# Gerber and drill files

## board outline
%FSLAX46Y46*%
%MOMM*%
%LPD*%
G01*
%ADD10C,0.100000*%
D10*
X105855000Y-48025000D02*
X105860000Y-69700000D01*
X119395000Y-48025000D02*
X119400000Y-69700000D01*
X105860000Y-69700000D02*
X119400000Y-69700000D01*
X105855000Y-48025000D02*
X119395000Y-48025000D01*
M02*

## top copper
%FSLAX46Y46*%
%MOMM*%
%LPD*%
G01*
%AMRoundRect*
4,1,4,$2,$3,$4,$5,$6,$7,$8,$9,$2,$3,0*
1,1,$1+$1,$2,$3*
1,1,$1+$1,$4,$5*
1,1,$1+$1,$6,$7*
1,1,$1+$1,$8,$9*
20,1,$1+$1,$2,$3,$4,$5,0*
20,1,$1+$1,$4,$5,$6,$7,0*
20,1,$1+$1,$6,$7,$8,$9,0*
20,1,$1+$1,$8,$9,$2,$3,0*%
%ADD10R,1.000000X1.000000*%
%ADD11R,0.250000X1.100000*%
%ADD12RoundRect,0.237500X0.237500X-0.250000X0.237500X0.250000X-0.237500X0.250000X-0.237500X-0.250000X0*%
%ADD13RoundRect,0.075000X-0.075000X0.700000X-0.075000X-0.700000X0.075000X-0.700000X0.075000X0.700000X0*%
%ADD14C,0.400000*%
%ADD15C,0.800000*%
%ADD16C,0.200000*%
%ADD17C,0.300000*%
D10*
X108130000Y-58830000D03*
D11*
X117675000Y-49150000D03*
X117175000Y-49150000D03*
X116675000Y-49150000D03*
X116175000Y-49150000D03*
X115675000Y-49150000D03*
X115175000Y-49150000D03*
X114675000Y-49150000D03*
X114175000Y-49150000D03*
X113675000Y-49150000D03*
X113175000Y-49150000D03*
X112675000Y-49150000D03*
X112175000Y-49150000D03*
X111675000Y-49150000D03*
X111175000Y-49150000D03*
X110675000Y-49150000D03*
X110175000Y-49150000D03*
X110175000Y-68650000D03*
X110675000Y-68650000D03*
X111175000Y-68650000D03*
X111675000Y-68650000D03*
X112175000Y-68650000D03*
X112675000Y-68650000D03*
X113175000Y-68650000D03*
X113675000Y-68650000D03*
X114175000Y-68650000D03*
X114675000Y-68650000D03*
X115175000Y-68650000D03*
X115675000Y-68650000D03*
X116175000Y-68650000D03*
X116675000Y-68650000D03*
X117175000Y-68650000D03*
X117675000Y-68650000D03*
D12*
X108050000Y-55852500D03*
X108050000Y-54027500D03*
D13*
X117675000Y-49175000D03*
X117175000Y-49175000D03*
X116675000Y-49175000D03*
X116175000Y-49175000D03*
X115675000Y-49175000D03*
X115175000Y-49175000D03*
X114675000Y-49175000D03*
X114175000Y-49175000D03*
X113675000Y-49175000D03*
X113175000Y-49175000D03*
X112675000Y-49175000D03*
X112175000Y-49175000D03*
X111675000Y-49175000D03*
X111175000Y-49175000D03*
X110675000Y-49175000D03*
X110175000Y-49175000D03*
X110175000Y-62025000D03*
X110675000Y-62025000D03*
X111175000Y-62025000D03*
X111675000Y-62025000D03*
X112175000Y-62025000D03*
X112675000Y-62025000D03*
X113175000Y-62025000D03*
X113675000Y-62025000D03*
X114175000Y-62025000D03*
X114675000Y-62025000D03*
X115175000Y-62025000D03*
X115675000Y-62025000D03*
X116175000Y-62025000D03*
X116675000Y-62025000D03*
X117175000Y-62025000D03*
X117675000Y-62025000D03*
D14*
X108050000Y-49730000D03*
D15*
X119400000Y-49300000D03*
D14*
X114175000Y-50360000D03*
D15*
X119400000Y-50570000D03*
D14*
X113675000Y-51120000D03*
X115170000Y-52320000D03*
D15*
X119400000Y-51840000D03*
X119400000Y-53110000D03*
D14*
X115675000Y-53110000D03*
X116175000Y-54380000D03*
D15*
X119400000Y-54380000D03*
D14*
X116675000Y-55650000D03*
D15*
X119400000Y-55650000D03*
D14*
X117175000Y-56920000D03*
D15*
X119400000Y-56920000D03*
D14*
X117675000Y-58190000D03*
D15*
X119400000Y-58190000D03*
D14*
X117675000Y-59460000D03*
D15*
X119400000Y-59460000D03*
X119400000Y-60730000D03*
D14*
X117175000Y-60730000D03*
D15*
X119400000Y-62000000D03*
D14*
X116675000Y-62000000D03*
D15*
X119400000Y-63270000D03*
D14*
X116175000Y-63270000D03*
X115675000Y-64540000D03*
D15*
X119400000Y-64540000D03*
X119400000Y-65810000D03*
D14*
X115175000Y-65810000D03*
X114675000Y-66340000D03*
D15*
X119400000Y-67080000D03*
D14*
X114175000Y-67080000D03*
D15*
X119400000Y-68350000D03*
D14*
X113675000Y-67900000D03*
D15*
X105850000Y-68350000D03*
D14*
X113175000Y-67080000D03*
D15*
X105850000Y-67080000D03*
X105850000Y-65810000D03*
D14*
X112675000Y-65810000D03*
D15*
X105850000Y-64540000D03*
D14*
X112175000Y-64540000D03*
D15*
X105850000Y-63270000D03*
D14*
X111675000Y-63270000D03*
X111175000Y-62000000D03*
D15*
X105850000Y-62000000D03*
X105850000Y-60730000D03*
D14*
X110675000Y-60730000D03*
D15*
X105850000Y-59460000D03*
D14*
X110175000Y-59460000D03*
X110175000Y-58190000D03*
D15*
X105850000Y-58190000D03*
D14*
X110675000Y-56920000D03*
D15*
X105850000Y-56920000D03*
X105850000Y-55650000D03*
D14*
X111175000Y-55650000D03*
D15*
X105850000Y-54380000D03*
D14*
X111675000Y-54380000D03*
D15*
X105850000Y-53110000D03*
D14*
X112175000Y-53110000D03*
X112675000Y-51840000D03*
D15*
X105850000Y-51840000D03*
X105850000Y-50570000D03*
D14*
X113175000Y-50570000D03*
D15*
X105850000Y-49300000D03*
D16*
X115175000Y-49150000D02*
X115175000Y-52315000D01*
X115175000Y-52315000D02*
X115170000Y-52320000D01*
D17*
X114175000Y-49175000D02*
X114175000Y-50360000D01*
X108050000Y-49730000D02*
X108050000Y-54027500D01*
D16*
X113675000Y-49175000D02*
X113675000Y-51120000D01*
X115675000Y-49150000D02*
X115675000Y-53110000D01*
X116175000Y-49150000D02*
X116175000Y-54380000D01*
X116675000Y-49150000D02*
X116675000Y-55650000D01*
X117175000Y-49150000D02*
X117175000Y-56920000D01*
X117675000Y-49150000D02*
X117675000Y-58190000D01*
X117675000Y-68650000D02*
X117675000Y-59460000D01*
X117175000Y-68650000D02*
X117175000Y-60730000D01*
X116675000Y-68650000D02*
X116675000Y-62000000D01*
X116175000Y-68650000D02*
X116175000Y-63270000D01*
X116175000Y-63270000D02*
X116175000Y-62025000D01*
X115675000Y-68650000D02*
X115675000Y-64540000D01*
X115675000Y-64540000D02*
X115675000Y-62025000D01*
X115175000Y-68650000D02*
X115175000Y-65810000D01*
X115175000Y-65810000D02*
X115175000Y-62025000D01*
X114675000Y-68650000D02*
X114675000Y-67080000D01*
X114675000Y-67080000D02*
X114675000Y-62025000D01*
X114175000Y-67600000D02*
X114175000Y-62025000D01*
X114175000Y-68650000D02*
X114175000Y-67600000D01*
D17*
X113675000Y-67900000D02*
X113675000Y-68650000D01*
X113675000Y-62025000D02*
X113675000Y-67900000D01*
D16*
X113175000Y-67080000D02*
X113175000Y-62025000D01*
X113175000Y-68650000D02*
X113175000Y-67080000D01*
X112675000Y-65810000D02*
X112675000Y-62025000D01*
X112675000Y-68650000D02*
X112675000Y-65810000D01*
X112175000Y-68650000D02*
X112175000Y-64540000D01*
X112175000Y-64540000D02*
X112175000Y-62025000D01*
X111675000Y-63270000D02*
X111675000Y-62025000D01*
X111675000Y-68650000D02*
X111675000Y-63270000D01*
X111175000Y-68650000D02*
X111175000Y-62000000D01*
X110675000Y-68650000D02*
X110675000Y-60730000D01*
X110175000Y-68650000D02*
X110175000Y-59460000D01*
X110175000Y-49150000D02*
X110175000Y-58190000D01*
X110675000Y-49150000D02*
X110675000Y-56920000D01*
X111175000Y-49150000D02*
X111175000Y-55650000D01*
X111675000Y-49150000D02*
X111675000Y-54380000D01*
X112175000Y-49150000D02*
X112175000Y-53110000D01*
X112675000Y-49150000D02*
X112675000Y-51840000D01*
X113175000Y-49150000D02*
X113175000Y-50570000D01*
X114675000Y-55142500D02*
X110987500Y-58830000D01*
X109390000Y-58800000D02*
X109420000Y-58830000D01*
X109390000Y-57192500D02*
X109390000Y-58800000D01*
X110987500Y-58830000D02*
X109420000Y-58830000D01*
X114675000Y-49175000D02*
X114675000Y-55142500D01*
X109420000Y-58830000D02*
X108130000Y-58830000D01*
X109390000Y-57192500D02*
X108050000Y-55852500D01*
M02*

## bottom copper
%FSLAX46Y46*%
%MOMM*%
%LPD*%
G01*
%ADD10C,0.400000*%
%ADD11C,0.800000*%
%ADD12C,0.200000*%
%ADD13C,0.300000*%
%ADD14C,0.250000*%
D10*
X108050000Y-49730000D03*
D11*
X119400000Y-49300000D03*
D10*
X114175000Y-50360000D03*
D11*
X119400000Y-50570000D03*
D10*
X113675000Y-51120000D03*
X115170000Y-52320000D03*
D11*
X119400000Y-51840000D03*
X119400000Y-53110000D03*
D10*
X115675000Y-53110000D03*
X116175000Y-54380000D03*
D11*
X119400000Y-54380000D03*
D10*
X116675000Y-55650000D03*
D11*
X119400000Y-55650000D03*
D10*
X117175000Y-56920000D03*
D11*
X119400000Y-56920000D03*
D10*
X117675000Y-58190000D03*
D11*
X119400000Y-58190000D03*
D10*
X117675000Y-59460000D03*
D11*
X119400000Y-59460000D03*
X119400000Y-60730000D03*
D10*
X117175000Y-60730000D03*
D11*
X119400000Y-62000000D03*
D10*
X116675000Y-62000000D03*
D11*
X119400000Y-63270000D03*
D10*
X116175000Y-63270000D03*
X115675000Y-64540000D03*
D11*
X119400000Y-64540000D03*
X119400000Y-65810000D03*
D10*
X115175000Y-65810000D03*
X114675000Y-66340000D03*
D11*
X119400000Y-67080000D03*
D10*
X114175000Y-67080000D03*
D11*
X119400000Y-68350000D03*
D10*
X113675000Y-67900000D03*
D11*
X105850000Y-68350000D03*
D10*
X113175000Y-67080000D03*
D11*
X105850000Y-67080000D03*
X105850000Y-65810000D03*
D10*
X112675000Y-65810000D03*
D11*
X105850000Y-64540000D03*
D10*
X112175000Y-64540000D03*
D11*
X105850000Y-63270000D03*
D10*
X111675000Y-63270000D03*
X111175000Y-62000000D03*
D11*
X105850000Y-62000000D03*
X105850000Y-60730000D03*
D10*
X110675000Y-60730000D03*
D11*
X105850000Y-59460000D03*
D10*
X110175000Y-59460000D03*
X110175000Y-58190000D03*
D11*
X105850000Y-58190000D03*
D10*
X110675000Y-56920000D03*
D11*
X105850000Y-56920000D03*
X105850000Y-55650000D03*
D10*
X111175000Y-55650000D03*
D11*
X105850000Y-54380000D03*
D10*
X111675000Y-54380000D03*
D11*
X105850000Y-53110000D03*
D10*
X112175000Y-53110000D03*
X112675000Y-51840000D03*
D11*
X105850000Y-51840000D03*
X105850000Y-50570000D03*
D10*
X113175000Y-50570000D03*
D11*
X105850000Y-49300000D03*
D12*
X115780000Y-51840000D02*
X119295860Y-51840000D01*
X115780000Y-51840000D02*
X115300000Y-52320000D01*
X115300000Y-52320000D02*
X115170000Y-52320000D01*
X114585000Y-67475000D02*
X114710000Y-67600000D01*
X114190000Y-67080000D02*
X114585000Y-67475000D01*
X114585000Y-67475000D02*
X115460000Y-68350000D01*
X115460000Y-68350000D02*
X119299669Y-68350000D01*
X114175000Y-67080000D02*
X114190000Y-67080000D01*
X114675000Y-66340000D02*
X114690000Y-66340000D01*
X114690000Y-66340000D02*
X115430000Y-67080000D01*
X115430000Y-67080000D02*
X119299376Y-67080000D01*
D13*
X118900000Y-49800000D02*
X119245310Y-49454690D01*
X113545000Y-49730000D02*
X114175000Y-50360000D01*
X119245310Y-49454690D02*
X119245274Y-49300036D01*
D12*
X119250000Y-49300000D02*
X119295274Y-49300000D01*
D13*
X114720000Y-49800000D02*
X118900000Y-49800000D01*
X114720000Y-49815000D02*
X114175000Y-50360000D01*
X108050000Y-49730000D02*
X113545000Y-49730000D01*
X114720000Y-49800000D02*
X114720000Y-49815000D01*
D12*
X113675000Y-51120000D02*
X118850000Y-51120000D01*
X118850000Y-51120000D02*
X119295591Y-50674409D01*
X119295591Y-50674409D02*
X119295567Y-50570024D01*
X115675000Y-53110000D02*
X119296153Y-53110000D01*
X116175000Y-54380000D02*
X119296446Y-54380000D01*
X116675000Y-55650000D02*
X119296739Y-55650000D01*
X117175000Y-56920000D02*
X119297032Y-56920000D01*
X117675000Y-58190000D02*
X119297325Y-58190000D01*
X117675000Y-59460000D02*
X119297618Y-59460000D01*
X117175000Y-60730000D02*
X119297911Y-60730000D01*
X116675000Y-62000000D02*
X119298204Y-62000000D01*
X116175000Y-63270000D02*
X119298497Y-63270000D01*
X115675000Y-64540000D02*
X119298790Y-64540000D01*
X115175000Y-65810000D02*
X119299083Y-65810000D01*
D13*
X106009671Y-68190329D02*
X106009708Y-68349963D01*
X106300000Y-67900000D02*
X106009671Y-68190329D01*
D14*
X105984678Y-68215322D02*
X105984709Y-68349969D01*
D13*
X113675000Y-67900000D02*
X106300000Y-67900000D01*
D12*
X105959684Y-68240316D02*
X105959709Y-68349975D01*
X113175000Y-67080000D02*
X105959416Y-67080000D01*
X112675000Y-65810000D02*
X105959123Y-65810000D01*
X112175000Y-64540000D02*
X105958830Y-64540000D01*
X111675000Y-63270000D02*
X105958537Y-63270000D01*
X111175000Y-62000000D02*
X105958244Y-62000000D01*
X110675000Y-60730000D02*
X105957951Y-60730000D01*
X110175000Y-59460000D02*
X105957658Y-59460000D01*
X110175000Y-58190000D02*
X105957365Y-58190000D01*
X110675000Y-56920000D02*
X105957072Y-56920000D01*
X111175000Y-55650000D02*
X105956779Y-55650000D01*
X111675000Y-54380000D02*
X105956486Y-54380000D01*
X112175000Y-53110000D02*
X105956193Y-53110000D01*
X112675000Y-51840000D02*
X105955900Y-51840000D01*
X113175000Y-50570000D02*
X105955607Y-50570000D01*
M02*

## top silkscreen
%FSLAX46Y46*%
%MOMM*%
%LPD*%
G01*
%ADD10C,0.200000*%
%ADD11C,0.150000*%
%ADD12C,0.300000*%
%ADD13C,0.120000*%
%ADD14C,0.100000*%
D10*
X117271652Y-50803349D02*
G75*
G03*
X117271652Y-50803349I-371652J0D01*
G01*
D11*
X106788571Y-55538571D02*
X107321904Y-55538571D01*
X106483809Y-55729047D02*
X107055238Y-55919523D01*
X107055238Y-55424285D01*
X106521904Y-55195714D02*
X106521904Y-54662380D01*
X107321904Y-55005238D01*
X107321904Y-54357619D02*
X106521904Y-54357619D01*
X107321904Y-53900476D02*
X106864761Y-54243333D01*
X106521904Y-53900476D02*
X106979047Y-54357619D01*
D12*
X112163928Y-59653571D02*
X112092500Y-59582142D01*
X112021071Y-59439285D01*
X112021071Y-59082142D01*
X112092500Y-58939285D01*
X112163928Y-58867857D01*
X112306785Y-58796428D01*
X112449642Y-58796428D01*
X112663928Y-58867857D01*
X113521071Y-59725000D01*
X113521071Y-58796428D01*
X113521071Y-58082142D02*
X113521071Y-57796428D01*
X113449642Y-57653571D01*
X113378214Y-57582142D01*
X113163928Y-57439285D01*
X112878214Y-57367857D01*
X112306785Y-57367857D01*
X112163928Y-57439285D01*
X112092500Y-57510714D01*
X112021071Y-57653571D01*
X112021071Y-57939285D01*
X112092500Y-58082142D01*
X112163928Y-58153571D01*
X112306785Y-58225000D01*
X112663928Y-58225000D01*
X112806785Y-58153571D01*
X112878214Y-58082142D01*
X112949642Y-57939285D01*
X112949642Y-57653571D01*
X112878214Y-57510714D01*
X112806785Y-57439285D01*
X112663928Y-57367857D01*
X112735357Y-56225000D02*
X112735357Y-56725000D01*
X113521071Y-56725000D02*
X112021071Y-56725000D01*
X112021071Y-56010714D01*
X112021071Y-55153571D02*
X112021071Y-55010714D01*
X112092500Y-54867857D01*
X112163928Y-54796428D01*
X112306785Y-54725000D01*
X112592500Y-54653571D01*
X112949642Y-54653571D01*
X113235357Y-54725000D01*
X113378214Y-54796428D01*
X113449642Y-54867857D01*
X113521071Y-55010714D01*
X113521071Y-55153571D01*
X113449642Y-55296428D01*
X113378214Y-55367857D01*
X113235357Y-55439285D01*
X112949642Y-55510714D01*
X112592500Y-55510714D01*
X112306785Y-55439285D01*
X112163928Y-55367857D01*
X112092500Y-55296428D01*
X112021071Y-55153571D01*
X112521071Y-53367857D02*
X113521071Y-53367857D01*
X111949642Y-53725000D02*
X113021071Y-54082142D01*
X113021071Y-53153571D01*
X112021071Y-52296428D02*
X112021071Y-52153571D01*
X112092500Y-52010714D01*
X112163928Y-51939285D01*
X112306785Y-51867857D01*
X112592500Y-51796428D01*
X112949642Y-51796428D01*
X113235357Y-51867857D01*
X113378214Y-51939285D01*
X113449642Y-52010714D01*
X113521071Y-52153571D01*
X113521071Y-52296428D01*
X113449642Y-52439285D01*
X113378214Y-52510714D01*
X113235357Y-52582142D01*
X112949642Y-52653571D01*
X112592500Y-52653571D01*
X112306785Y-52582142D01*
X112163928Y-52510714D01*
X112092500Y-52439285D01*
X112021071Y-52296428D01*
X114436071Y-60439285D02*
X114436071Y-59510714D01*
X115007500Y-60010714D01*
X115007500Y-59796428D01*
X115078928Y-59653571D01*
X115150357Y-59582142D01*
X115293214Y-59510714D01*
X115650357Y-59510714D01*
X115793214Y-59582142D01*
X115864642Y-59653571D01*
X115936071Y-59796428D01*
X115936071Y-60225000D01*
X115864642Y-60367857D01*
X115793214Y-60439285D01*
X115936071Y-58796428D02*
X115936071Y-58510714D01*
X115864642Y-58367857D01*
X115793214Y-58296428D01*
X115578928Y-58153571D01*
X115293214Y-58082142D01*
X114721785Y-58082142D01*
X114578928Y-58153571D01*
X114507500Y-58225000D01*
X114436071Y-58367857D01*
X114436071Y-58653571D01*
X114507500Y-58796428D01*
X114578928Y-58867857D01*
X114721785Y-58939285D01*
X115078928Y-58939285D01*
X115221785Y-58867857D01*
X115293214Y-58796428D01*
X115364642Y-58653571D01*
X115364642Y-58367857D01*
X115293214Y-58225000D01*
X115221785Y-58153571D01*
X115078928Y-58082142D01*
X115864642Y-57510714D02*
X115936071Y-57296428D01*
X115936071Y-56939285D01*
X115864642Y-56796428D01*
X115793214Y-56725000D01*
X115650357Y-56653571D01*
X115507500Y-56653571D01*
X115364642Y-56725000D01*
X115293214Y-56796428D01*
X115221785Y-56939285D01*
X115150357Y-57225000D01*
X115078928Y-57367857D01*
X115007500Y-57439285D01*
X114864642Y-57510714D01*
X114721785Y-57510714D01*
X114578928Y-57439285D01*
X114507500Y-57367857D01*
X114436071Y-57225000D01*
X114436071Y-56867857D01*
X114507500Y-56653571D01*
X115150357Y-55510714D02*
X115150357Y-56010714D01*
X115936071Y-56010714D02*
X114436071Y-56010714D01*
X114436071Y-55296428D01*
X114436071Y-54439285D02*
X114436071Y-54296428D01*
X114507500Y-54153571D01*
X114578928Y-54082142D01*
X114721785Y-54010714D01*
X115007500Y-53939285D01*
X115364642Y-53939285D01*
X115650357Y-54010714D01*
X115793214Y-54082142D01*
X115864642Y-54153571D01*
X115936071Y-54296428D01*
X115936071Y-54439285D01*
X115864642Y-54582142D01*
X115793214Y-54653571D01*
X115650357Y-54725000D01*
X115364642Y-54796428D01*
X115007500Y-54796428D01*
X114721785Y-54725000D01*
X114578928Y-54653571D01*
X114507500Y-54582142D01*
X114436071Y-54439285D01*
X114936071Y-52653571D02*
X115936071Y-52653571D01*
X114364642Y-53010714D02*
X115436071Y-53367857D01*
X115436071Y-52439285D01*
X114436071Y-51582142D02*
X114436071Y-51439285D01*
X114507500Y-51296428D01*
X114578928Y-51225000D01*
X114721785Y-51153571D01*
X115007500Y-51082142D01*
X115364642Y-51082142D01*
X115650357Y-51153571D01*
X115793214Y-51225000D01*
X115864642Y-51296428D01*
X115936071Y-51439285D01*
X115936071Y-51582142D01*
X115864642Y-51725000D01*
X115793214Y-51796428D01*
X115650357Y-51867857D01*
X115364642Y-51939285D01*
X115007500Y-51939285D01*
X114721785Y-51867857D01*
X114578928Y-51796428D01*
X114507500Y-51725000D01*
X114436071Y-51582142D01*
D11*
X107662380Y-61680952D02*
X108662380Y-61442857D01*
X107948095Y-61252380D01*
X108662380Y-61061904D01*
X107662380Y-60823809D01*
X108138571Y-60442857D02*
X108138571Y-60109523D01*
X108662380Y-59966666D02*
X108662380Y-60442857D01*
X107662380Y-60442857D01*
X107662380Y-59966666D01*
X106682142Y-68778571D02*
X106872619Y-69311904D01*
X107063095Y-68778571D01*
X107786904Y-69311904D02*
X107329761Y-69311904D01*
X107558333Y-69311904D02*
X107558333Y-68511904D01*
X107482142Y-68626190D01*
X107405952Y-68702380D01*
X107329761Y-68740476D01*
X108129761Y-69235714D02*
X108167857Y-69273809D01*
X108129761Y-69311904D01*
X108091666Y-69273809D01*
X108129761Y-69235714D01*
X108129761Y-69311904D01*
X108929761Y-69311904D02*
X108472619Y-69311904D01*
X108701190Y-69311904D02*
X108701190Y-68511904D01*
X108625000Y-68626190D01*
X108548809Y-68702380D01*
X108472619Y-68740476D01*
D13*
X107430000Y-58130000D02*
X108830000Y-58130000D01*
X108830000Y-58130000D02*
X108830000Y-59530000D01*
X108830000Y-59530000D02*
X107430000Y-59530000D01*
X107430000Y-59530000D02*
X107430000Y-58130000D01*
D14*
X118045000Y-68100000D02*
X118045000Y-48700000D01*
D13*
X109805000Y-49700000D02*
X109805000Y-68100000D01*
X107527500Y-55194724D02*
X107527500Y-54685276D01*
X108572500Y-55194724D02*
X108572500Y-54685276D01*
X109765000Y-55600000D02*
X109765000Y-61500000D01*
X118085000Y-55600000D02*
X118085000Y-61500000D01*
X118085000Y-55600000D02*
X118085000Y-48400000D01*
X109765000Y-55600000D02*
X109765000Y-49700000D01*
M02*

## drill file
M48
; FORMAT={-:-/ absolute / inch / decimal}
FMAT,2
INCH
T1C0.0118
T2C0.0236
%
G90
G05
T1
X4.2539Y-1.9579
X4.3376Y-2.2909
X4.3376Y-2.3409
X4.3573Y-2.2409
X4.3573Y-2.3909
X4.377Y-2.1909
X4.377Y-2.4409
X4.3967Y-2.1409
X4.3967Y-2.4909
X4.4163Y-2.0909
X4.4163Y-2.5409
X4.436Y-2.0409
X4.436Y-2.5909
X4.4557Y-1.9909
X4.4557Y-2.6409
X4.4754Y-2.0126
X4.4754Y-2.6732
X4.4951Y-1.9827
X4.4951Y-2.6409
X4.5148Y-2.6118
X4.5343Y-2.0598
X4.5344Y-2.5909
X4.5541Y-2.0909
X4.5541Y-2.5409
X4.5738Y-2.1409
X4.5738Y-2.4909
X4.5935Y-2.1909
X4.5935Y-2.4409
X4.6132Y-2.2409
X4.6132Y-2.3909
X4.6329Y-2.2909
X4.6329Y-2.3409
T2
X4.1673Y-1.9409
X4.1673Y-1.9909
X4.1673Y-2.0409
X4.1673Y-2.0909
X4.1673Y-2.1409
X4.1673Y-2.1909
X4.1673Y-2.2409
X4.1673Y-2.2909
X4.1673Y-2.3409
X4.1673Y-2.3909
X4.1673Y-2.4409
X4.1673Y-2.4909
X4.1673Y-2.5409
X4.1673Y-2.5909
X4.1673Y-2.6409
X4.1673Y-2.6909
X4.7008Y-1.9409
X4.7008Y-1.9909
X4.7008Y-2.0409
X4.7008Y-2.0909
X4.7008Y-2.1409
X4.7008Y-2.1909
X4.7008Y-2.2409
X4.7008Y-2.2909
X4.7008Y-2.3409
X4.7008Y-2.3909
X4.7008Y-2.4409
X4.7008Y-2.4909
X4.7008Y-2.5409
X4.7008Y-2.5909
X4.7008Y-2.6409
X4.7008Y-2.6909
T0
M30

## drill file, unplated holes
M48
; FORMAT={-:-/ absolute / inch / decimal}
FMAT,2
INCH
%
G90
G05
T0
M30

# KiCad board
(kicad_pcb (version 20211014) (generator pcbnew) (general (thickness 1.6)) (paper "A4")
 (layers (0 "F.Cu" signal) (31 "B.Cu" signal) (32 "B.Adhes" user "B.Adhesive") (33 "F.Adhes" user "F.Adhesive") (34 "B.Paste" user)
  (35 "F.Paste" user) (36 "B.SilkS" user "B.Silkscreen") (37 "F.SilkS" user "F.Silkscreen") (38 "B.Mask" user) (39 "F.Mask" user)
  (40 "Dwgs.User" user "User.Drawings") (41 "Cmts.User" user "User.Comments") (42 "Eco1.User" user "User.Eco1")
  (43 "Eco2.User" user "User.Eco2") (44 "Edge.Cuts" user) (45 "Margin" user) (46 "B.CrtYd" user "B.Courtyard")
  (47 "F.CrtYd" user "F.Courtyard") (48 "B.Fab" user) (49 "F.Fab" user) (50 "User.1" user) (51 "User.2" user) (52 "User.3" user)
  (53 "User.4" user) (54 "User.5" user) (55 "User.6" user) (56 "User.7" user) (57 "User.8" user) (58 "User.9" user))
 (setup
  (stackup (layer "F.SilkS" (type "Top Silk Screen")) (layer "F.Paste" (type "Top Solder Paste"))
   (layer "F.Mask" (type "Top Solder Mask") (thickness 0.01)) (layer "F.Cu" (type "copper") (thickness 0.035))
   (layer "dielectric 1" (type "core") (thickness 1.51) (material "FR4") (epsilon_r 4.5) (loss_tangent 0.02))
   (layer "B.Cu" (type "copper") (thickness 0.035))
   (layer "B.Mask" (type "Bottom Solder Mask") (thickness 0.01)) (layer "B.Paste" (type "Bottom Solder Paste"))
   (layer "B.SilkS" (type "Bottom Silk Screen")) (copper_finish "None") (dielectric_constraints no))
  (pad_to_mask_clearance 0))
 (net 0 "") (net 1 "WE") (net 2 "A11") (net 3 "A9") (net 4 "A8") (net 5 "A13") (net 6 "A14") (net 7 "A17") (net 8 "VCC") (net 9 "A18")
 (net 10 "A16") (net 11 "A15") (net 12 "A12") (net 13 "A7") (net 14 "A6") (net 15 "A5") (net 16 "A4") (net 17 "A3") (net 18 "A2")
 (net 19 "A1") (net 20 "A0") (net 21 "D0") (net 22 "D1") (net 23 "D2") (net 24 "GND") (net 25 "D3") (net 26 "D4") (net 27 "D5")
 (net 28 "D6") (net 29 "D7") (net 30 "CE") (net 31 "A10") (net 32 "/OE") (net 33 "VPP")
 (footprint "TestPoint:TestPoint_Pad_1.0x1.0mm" (layer "F.Cu") (at 108.13 58.83)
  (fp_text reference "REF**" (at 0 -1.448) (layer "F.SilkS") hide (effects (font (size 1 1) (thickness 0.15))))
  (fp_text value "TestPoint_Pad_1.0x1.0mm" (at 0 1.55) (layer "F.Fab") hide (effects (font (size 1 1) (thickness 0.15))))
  (fp_line (start -0.7 -0.7) (end 0.7 -0.7) (layer "F.SilkS") (width 0.12))
  (fp_line (start 0.7 -0.7) (end 0.7 0.7) (layer "F.SilkS") (width 0.12))
  (fp_line (start 0.7 0.7) (end -0.7 0.7) (layer "F.SilkS") (width 0.12))
  (fp_line (start -0.7 0.7) (end -0.7 -0.7) (layer "F.SilkS") (width 0.12))
  (pad "" smd rect (at 0 0) (size 1 1) (layers "F.Cu" "F.Mask") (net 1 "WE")))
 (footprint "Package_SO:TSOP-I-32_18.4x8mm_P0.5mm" (layer "F.Cu") (at 113.925 58.9 -90)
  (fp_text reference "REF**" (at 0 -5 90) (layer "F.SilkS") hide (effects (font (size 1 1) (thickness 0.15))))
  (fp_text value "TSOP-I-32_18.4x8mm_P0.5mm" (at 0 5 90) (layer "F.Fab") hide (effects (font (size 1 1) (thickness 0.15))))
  (fp_line (start 9.2 -4.12) (end -10.2 -4.12) (layer "F.SilkS") (width 0.1))
  (fp_line (start -9.2 4.12) (end 9.2 4.12) (layer "F.SilkS") (width 0.12))
  (pad "1" smd rect (at -9.75 -3.75 270) (size 1.1 0.25) (layers "F.Cu" "F.Paste" "F.Mask") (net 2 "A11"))
  (pad "2" smd rect (at -9.75 -3.25 270) (size 1.1 0.25) (layers "F.Cu" "F.Paste" "F.Mask") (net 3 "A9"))
  (pad "3" smd rect (at -9.75 -2.75 270) (size 1.1 0.25) (layers "F.Cu" "F.Paste" "F.Mask") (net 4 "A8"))
  (pad "4" smd rect (at -9.75 -2.25 270) (size 1.1 0.25) (layers "F.Cu" "F.Paste" "F.Mask") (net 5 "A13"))
  (pad "5" smd rect (at -9.75 -1.75 270) (size 1.1 0.25) (layers "F.Cu" "F.Paste" "F.Mask") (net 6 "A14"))
  (pad "6" smd rect (at -9.75 -1.25 270) (size 1.1 0.25) (layers "F.Cu" "F.Paste" "F.Mask") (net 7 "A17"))
  (pad "7" smd rect (at -9.75 -0.75 270) (size 1.1 0.25) (layers "F.Cu" "F.Paste" "F.Mask") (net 1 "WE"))
  (pad "8" smd rect (at -9.75 -0.25 270) (size 1.1 0.25) (layers "F.Cu" "F.Paste" "F.Mask") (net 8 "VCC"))
  (pad "9" smd rect (at -9.75 0.25 270) (size 1.1 0.25) (layers "F.Cu" "F.Paste" "F.Mask") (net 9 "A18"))
  (pad "10" smd rect (at -9.75 0.75 270) (size 1.1 0.25) (layers "F.Cu" "F.Paste" "F.Mask") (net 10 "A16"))
  (pad "11" smd rect (at -9.75 1.25 270) (size 1.1 0.25) (layers "F.Cu" "F.Paste" "F.Mask") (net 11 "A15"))
  (pad "12" smd rect (at -9.75 1.75 270) (size 1.1 0.25) (layers "F.Cu" "F.Paste" "F.Mask") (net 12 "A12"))
  (pad "13" smd rect (at -9.75 2.25 270) (size 1.1 0.25) (layers "F.Cu" "F.Paste" "F.Mask") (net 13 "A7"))
  (pad "14" smd rect (at -9.75 2.75 270) (size 1.1 0.25) (layers "F.Cu" "F.Paste" "F.Mask") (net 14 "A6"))
  (pad "15" smd rect (at -9.75 3.25 270) (size 1.1 0.25) (layers "F.Cu" "F.Paste" "F.Mask") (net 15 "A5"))
  (pad "16" smd rect (at -9.75 3.75 270) (size 1.1 0.25) (layers "F.Cu" "F.Paste" "F.Mask") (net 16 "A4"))
  (pad "17" smd rect (at 9.75 3.75 270) (size 1.1 0.25) (layers "F.Cu" "F.Paste" "F.Mask") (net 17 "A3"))
  (pad "18" smd rect (at 9.75 3.25 270) (size 1.1 0.25) (layers "F.Cu" "F.Paste" "F.Mask") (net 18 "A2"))
  (pad "19" smd rect (at 9.75 2.75 270) (size 1.1 0.25) (layers "F.Cu" "F.Paste" "F.Mask") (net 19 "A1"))
  (pad "20" smd rect (at 9.75 2.25 270) (size 1.1 0.25) (layers "F.Cu" "F.Paste" "F.Mask") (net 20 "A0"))
  (pad "21" smd rect (at 9.75 1.75 270) (size 1.1 0.25) (layers "F.Cu" "F.Paste" "F.Mask") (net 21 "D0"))
  (pad "22" smd rect (at 9.75 1.25 270) (size 1.1 0.25) (layers "F.Cu" "F.Paste" "F.Mask") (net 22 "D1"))
  (pad "23" smd rect (at 9.75 0.75 270) (size 1.1 0.25) (layers "F.Cu" "F.Paste" "F.Mask") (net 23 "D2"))
  (pad "24" smd rect (at 9.75 0.25 270) (size 1.1 0.25) (layers "F.Cu" "F.Paste" "F.Mask") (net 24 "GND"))
  (pad "25" smd rect (at 9.75 -0.25 270) (size 1.1 0.25) (layers "F.Cu" "F.Paste" "F.Mask") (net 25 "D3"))
  (pad "26" smd rect (at 9.75 -0.75 270) (size 1.1 0.25) (layers "F.Cu" "F.Paste" "F.Mask") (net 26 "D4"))
  (pad "27" smd rect (at 9.75 -1.25 270) (size 1.1 0.25) (layers "F.Cu" "F.Paste" "F.Mask") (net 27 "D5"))
  (pad "28" smd rect (at 9.75 -1.75 270) (size 1.1 0.25) (layers "F.Cu" "F.Paste" "F.Mask") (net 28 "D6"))
  (pad "29" smd rect (at 9.75 -2.25 270) (size 1.1 0.25) (layers "F.Cu" "F.Paste" "F.Mask") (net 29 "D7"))
  (pad "30" smd rect (at 9.75 -2.75 270) (size 1.1 0.25) (layers "F.Cu" "F.Paste" "F.Mask") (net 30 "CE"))
  (pad "31" smd rect (at 9.75 -3.25 270) (size 1.1 0.25) (layers "F.Cu" "F.Paste" "F.Mask") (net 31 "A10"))
  (pad "32" smd rect (at 9.75 -3.75 270) (size 1.1 0.25) (layers "F.Cu" "F.Paste" "F.Mask") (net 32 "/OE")))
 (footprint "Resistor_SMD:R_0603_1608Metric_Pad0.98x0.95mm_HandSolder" (layer "F.Cu") (at 108.05 54.94 90)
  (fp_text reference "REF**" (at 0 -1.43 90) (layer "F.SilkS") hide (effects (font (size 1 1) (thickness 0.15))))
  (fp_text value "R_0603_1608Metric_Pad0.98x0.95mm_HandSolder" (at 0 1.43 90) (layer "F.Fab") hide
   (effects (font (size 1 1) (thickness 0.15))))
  (fp_line (start -0.254724 -0.5225) (end 0.254724 -0.5225) (layer "F.SilkS") (width 0.12))
  (fp_line (start -0.254724 0.5225) (end 0.254724 0.5225) (layer "F.SilkS") (width 0.12))
  (pad "" smd roundrect (at -0.9125 0 90) (size 0.975 0.95) (layers "F.Cu" "F.Paste" "F.Mask") (roundrect_rratio 0.25) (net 1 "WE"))
  (pad "" smd roundrect (at 0.9125 0 90) (size 0.975 0.95) (layers "F.Cu" "F.Paste" "F.Mask") (roundrect_rratio 0.25) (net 8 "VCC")))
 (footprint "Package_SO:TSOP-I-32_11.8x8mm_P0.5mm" (layer "F.Cu") (at 113.925 55.6 -90)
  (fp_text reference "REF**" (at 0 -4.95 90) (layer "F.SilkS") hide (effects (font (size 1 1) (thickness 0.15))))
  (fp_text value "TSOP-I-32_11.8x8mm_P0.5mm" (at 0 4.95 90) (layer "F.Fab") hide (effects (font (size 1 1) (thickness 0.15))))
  (fp_line (start 0 4.16) (end 5.9 4.16) (layer "F.SilkS") (width 0.12))
  (fp_line (start 0 -4.16) (end 5.9 -4.16) (layer "F.SilkS") (width 0.12))
  (fp_line (start 0 -4.16) (end -7.2 -4.16) (layer "F.SilkS") (width 0.12))
  (fp_line (start 0 4.16) (end -5.9 4.16) (layer "F.SilkS") (width 0.12))
  (pad "1" smd roundrect (at -6.425 -3.75 270) (size 1.55 0.3) (layers "F.Cu" "F.Paste" "F.Mask") (roundrect_rratio 0.25))
  (pad "2" smd roundrect (at -6.425 -3.25 270) (size 1.55 0.3) (layers "F.Cu" "F.Paste" "F.Mask") (roundrect_rratio 0.25))
  (pad "3" smd roundrect (at -6.425 -2.75 270) (size 1.55 0.3) (layers "F.Cu" "F.Paste" "F.Mask") (roundrect_rratio 0.25))
  (pad "4" smd roundrect (at -6.425 -2.25 270) (size 1.55 0.3) (layers "F.Cu" "F.Paste" "F.Mask") (roundrect_rratio 0.25))
  (pad "5" smd roundrect (at -6.425 -1.75 270) (size 1.55 0.3) (layers "F.Cu" "F.Paste" "F.Mask") (roundrect_rratio 0.25))
  (pad "6" smd roundrect (at -6.425 -1.25 270) (size 1.55 0.3) (layers "F.Cu" "F.Paste" "F.Mask") (roundrect_rratio 0.25))
  (pad "7" smd roundrect (at -6.425 -0.75 270) (size 1.55 0.3) (layers "F.Cu" "F.Paste" "F.Mask") (roundrect_rratio 0.25) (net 1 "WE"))
  (pad "8" smd roundrect (at -6.425 -0.25 270) (size 1.55 0.3) (layers "F.Cu" "F.Paste" "F.Mask") (roundrect_rratio 0.25) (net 8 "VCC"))
  (pad "9" smd roundrect (at -6.425 0.25 270) (size 1.55 0.3) (layers "F.Cu" "F.Paste" "F.Mask") (roundrect_rratio 0.25) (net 9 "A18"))
  (pad "10" smd roundrect (at -6.425 0.75 270) (size 1.55 0.3) (layers "F.Cu" "F.Paste" "F.Mask") (roundrect_rratio 0.25))
  (pad "11" smd roundrect (at -6.425 1.25 270) (size 1.55 0.3) (layers "F.Cu" "F.Paste" "F.Mask") (roundrect_rratio 0.25))
  (pad "12" smd roundrect (at -6.425 1.75 270) (size 1.55 0.3) (layers "F.Cu" "F.Paste" "F.Mask") (roundrect_rratio 0.25))
  (pad "13" smd roundrect (at -6.425 2.25 270) (size 1.55 0.3) (layers "F.Cu" "F.Paste" "F.Mask") (roundrect_rratio 0.25))
  (pad "14" smd roundrect (at -6.425 2.75 270) (size 1.55 0.3) (layers "F.Cu" "F.Paste" "F.Mask") (roundrect_rratio 0.25))
  (pad "15" smd roundrect (at -6.425 3.25 270) (size 1.55 0.3) (layers "F.Cu" "F.Paste" "F.Mask") (roundrect_rratio 0.25))
  (pad "16" smd roundrect (at -6.425 3.75 270) (size 1.55 0.3) (layers "F.Cu" "F.Paste" "F.Mask") (roundrect_rratio 0.25))
  (pad "17" smd roundrect (at 6.425 3.75 270) (size 1.55 0.3) (layers "F.Cu" "F.Paste" "F.Mask") (roundrect_rratio 0.25) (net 17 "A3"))
  (pad "18" smd roundrect (at 6.425 3.25 270) (size 1.55 0.3) (layers "F.Cu" "F.Paste" "F.Mask") (roundrect_rratio 0.25) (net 18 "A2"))
  (pad "19" smd roundrect (at 6.425 2.75 270) (size 1.55 0.3) (layers "F.Cu" "F.Paste" "F.Mask") (roundrect_rratio 0.25) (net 19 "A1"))
  (pad "20" smd roundrect (at 6.425 2.25 270) (size 1.55 0.3) (layers "F.Cu" "F.Paste" "F.Mask") (roundrect_rratio 0.25) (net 20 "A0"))
  (pad "21" smd roundrect (at 6.425 1.75 270) (size 1.55 0.3) (layers "F.Cu" "F.Paste" "F.Mask") (roundrect_rratio 0.25) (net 21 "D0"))
  (pad "22" smd roundrect (at 6.425 1.25 270) (size 1.55 0.3) (layers "F.Cu" "F.Paste" "F.Mask") (roundrect_rratio 0.25) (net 22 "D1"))
  (pad "23" smd roundrect (at 6.425 0.75 270) (size 1.55 0.3) (layers "F.Cu" "F.Paste" "F.Mask") (roundrect_rratio 0.25) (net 23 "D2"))
  (pad "24" smd roundrect (at 6.425 0.25 270) (size 1.55 0.3) (layers "F.Cu" "F.Paste" "F.Mask") (roundrect_rratio 0.25) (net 24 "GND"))
  (pad "25" smd roundrect (at 6.425 -0.25 270) (size 1.55 0.3) (layers "F.Cu" "F.Paste" "F.Mask") (roundrect_rratio 0.25) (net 25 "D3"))
  (pad "26" smd roundrect (at 6.425 -0.75 270) (size 1.55 0.3) (layers "F.Cu" "F.Paste" "F.Mask") (roundrect_rratio 0.25) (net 26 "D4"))
  (pad "27" smd roundrect (at 6.425 -1.25 270) (size 1.55 0.3) (layers "F.Cu" "F.Paste" "F.Mask") (roundrect_rratio 0.25) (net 27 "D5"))
  (pad "28" smd roundrect (at 6.425 -1.75 270) (size 1.55 0.3) (layers "F.Cu" "F.Paste" "F.Mask") (roundrect_rratio 0.25) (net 28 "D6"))
  (pad "29" smd roundrect (at 6.425 -2.25 270) (size 1.55 0.3) (layers "F.Cu" "F.Paste" "F.Mask") (roundrect_rratio 0.25) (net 29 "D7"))
  (pad "30" smd roundrect (at 6.425 -2.75 270) (size 1.55 0.3) (layers "F.Cu" "F.Paste" "F.Mask") (roundrect_rratio 0.25) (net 30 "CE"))
  (pad "31" smd roundrect (at 6.425 -3.25 270) (size 1.55 0.3) (layers "F.Cu" "F.Paste" "F.Mask") (roundrect_rratio 0.25) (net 31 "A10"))
  (pad "32" smd roundrect (at 6.425 -3.75 270) (size 1.55 0.3) (layers "F.Cu" "F.Paste" "F.Mask") (roundrect_rratio 0.25) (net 32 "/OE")))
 (gr_circle (center 116.9 50.803349) (end 117.25 50.928349) (layer "F.SilkS") (width 0.2) (fill none))
 (gr_line (start 105.855 48.025) (end 105.86 69.7) (layer "Edge.Cuts") (width 0.1))
 (gr_line (start 119.395 48.025) (end 119.4 69.7) (layer "Edge.Cuts") (width 0.1))
 (gr_line (start 105.86 69.7) (end 119.4 69.7) (layer "Edge.Cuts") (width 0.1))
 (gr_line (start 105.855 48.025) (end 119.395 48.025) (layer "Edge.Cuts") (width 0.1))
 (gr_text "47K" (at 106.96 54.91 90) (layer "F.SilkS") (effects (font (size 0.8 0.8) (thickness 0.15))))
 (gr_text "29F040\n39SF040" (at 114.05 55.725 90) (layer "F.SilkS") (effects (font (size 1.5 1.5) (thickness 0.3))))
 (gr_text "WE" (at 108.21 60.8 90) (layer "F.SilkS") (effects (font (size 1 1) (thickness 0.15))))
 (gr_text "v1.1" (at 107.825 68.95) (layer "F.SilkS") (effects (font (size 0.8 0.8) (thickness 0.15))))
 (segment (start 114.175 49.175) (end 114.175 50.36) (width 0.3) (layer "F.Cu") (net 8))
 (segment (start 108.05 49.73) (end 108.05 54.0275) (width 0.3) (layer "F.Cu") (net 8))
 (via (at 108.05 49.73) (size 0.4) (drill 0.3) (layers "F.Cu" "B.Cu") (free) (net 8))
 (via (at 119.4 49.3) (size 0.8) (drill 0.6) (layers "F.Cu" "B.Cu") (free) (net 8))
 (via (at 114.175 50.36) (size 0.4) (drill 0.3) (layers "F.Cu" "B.Cu") (free) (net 8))
 (segment (start 118.9 49.8) (end 119.24531 49.45469) (width 0.3) (layer "B.Cu") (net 8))
 (segment (start 113.545 49.73) (end 114.175 50.36) (width 0.3) (layer "B.Cu") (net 8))
 (segment (start 119.24531 49.45469) (end 119.245274 49.300036) (width 0.3) (layer "B.Cu") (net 8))
 (segment (start 119.25 49.3) (end 119.295274 49.3) (width 0.2) (layer "B.Cu") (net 8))
 (segment (start 114.72 49.8) (end 118.9 49.8) (width 0.3) (layer "B.Cu") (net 8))
 (segment (start 114.72 49.815) (end 114.175 50.36) (width 0.3) (layer "B.Cu") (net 8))
 (segment (start 108.05 49.73) (end 113.545 49.73) (width 0.3) (layer "B.Cu") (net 8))
 (segment (start 114.72 49.8) (end 114.72 49.815) (width 0.3) (layer "B.Cu") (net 8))
 (segment (start 113.675 49.175) (end 113.675 51.12) (width 0.2) (layer "F.Cu") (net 9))
 (via (at 119.4 50.57) (size 0.8) (drill 0.6) (layers "F.Cu" "B.Cu") (free) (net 9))
 (via (at 113.675 51.12) (size 0.4) (drill 0.3) (layers "F.Cu" "B.Cu") (free) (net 9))
 (segment (start 113.675 51.12) (end 118.85 51.12) (width 0.2) (layer "B.Cu") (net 9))
 (segment (start 118.85 51.12) (end 119.295591 50.674409) (width 0.2) (layer "B.Cu") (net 9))
 (segment (start 119.295591 50.674409) (end 119.295567 50.570024) (width 0.2) (layer "B.Cu") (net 9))
 (segment (start 115.175 52.315) (end 115.17 52.32) (width 0.2) (layer "F.Cu") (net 7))
 (segment (start 115.175 49.15) (end 115.175 52.315) (width 0.2) (layer "F.Cu") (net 7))
 (via (at 115.17 52.32) (size 0.4) (drill 0.3) (layers "F.Cu" "B.Cu") (free) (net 7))
 (via (at 119.4 51.84) (size 0.8) (drill 0.6) (layers "F.Cu" "B.Cu") (free) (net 7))
 (segment (start 115.78 51.84) (end 115.3 52.32) (width 0.2) (layer "B.Cu") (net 7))
 (segment (start 115.78 51.84) (end 119.29586 51.84) (width 0.2) (layer "B.Cu") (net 7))
 (segment (start 115.3 52.32) (end 115.17 52.32) (width 0.2) (layer "B.Cu") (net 7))
 (segment (start 115.675 49.15) (end 115.675 53.11) (width 0.2) (layer "F.Cu") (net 6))
 (via (at 119.4 53.11) (size 0.8) (drill 0.6) (layers "F.Cu" "B.Cu") (free) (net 6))
 (via (at 115.675 53.11) (size 0.4) (drill 0.3) (layers "F.Cu" "B.Cu") (free) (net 6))
 (segment (start 115.675 53.11) (end 119.296153 53.11) (width 0.2) (layer "B.Cu") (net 6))
 (segment (start 116.175 49.15) (end 116.175 54.38) (width 0.2) (layer "F.Cu") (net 5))
 (via (at 116.175 54.38) (size 0.4) (drill 0.3) (layers "F.Cu" "B.Cu") (free) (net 5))
 (via (at 119.4 54.38) (size 0.8) (drill 0.6) (layers "F.Cu" "B.Cu") (free) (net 5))
 (segment (start 116.175 54.38) (end 119.296446 54.38) (width 0.2) (layer "B.Cu") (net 5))
 (segment (start 116.675 49.15) (end 116.675 55.65) (width 0.2) (layer "F.Cu") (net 4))
 (via (at 116.675 55.65) (size 0.4) (drill 0.3) (layers "F.Cu" "B.Cu") (free) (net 4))
 (via (at 119.4 55.65) (size 0.8) (drill 0.6) (layers "F.Cu" "B.Cu") (free) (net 4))
 (segment (start 116.675 55.65) (end 119.296739 55.65) (width 0.2) (layer "B.Cu") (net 4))
 (segment (start 117.175 49.15) (end 117.175 56.92) (width 0.2) (layer "F.Cu") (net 3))
 (via (at 117.175 56.92) (size 0.4) (drill 0.3) (layers "F.Cu" "B.Cu") (free) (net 3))
 (via (at 119.4 56.92) (size 0.8) (drill 0.6) (layers "F.Cu" "B.Cu") (free) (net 3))
 (segment (start 117.175 56.92) (end 119.297032 56.92) (width 0.2) (layer "B.Cu") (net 3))
 (segment (start 117.675 49.15) (end 117.675 58.19) (width 0.2) (layer "F.Cu") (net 2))
 (via (at 117.675 58.19) (size 0.4) (drill 0.3) (layers "F.Cu" "B.Cu") (free) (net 2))
 (via (at 119.4 58.19) (size 0.8) (drill 0.6) (layers "F.Cu" "B.Cu") (free) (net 2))
 (segment (start 117.675 58.19) (end 119.297325 58.19) (width 0.2) (layer "B.Cu") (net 2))
 (segment (start 117.675 68.65) (end 117.675 59.46) (width 0.2) (layer "F.Cu") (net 32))
 (via (at 117.675 59.46) (size 0.4) (drill 0.3) (layers "F.Cu" "B.Cu") (free) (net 32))
 (via (at 119.4 59.46) (size 0.8) (drill 0.6) (layers "F.Cu" "B.Cu") (free) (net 32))
 (segment (start 117.675 59.46) (end 119.297618 59.46) (width 0.2) (layer "B.Cu") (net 32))
 (segment (start 117.175 68.65) (end 117.175 60.73) (width 0.2) (layer "F.Cu") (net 31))
 (via (at 119.4 60.73) (size 0.8) (drill 0.6) (layers "F.Cu" "B.Cu") (free) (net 31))
 (via (at 117.175 60.73) (size 0.4) (drill 0.3) (layers "F.Cu" "B.Cu") (free) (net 31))
 (segment (start 117.175 60.73) (end 119.297911 60.73) (width 0.2) (layer "B.Cu") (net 31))
 (segment (start 116.675 68.65) (end 116.675 62) (width 0.2) (layer "F.Cu") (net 30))
 (via (at 119.4 62) (size 0.8) (drill 0.6) (layers "F.Cu" "B.Cu") (free) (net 30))
 (via (at 116.675 62) (size 0.4) (drill 0.3) (layers "F.Cu" "B.Cu") (free) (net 30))
 (segment (start 116.675 62) (end 119.298204 62) (width 0.2) (layer "B.Cu") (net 30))
 (segment (start 116.175 68.65) (end 116.175 63.27) (width 0.2) (layer "F.Cu") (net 29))
 (segment (start 116.175 63.27) (end 116.175 62.025) (width 0.2) (layer "F.Cu") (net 29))
 (via (at 119.4 63.27) (size 0.8) (drill 0.6) (layers "F.Cu" "B.Cu") (free) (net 29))
 (via (at 116.175 63.27) (size 0.4) (drill 0.3) (layers "F.Cu" "B.Cu") (free) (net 29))
 (segment (start 116.175 63.27) (end 119.298497 63.27) (width 0.2) (layer "B.Cu") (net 29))
 (segment (start 115.675 68.65) (end 115.675 64.54) (width 0.2) (layer "F.Cu") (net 28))
 (segment (start 115.675 64.54) (end 115.675 62.025) (width 0.2) (layer "F.Cu") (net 28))
 (via (at 115.675 64.54) (size 0.4) (drill 0.3) (layers "F.Cu" "B.Cu") (free) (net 28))
 (via (at 119.4 64.54) (size 0.8) (drill 0.6) (layers "F.Cu" "B.Cu") (free) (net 28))
 (segment (start 115.675 64.54) (end 119.29879 64.54) (width 0.2) (layer "B.Cu") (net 28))
 (segment (start 115.175 68.65) (end 115.175 65.81) (width 0.2) (layer "F.Cu") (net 27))
 (segment (start 115.175 65.81) (end 115.175 62.025) (width 0.2) (layer "F.Cu") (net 27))
 (via (at 119.4 65.81) (size 0.8) (drill 0.6) (layers "F.Cu" "B.Cu") (free) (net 27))
 (via (at 115.175 65.81) (size 0.4) (drill 0.3) (layers "F.Cu" "B.Cu") (free) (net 27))
 (segment (start 115.175 65.81) (end 119.299083 65.81) (width 0.2) (layer "B.Cu") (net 27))
 (segment (start 114.675 68.65) (end 114.675 67.08) (width 0.2) (layer "F.Cu") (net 26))
 (segment (start 114.675 67.08) (end 114.675 62.025) (width 0.2) (layer "F.Cu") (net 26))
 (via (at 114.675 66.34) (size 0.4) (drill 0.3) (layers "F.Cu" "B.Cu") (free) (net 26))
 (via (at 119.4 67.08) (size 0.8) (drill 0.6) (layers "F.Cu" "B.Cu") (free) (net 26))
 (segment (start 114.675 66.34) (end 114.69 66.34) (width 0.2) (layer "B.Cu") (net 26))
 (segment (start 114.69 66.34) (end 115.43 67.08) (width 0.2) (layer "B.Cu") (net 26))
 (segment (start 115.43 67.08) (end 119.299376 67.08) (width 0.2) (layer "B.Cu") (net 26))
 (segment (start 114.175 67.6) (end 114.175 62.025) (width 0.2) (layer "F.Cu") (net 25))
 (segment (start 114.175 68.65) (end 114.175 67.6) (width 0.2) (layer "F.Cu") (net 25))
 (via (at 114.175 67.08) (size 0.4) (drill 0.3) (layers "F.Cu" "B.Cu") (free) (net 25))
 (via (at 119.4 68.35) (size 0.8) (drill 0.6) (layers "F.Cu" "B.Cu") (free) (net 25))
 (segment (start 114.585 67.475) (end 115.46 68.35) (width 0.2) (layer "B.Cu") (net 25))
 (segment (start 114.175 67.08) (end 114.19 67.08) (width 0.2) (layer "B.Cu") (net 25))
 (segment (start 114.19 67.08) (end 114.585 67.475) (width 0.2) (layer "B.Cu") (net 25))
 (segment (start 115.46 68.35) (end 119.299669 68.35) (width 0.2) (layer "B.Cu") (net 25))
 (segment (start 114.585 67.475) (end 114.71 67.6) (width 0.2) (layer "B.Cu") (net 25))
 (segment (start 113.675 67.9) (end 113.675 68.65) (width 0.3) (layer "F.Cu") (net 24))
 (segment (start 113.675 62.025) (end 113.675 67.9) (width 0.3) (layer "F.Cu") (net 24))
 (via (at 113.675 67.9) (size 0.4) (drill 0.3) (layers "F.Cu" "B.Cu") (free) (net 24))
 (via (at 105.85 68.35) (size 0.8) (drill 0.6) (layers "F.Cu" "B.Cu") (free) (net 24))
 (segment (start 106.009671 68.190329) (end 106.009708 68.349963) (width 0.3) (layer "B.Cu") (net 24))
 (segment (start 106.3 67.9) (end 106.009671 68.190329) (width 0.3) (layer "B.Cu") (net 24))
 (segment (start 105.984678 68.215322) (end 105.984709 68.349969) (width 0.25) (layer "B.Cu") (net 24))
 (segment (start 113.675 67.9) (end 106.3 67.9) (width 0.3) (layer "B.Cu") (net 24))
 (segment (start 105.959684 68.240316) (end 105.959709 68.349975) (width 0.2) (layer "B.Cu") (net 24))
 (segment (start 113.175 67.08) (end 113.175 62.025) (width 0.2) (layer "F.Cu") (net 23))
 (segment (start 113.175 68.65) (end 113.175 67.08) (width 0.2) (layer "F.Cu") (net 23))
 (via (at 113.175 67.08) (size 0.4) (drill 0.3) (layers "F.Cu" "B.Cu") (free) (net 23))
 (via (at 105.85 67.08) (size 0.8) (drill 0.6) (layers "F.Cu" "B.Cu") (free) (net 23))
 (segment (start 113.175 67.08) (end 105.959416 67.08) (width 0.2) (layer "B.Cu") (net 23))
 (segment (start 112.675 65.81) (end 112.675 62.025) (width 0.2) (layer "F.Cu") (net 22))
 (segment (start 112.675 68.65) (end 112.675 65.81) (width 0.2) (layer "F.Cu") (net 22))
 (via (at 105.85 65.81) (size 0.8) (drill 0.6) (layers "F.Cu" "B.Cu") (free) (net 22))
 (via (at 112.675 65.81) (size 0.4) (drill 0.3) (layers "F.Cu" "B.Cu") (free) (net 22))
 (segment (start 112.675 65.81) (end 105.959123 65.81) (width 0.2) (layer "B.Cu") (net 22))
 (segment (start 112.175 68.65) (end 112.175 64.54) (width 0.2) (layer "F.Cu") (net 21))
 (segment (start 112.175 64.54) (end 112.175 62.025) (width 0.2) (layer "F.Cu") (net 21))
 (via (at 105.85 64.54) (size 0.8) (drill 0.6) (layers "F.Cu" "B.Cu") (free) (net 21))
 (via (at 112.175 64.54) (size 0.4) (drill 0.3) (layers "F.Cu" "B.Cu") (free) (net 21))
 (segment (start 112.175 64.54) (end 105.95883 64.54) (width 0.2) (layer "B.Cu") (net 21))
 (segment (start 111.675 63.27) (end 111.675 62.025) (width 0.2) (layer "F.Cu") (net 20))
 (segment (start 111.675 68.65) (end 111.675 63.27) (width 0.2) (layer "F.Cu") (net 20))
 (via (at 105.85 63.27) (size 0.8) (drill 0.6) (layers "F.Cu" "B.Cu") (free) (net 20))
 (via (at 111.675 63.27) (size 0.4) (drill 0.3) (layers "F.Cu" "B.Cu") (free) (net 20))
 (segment (start 111.675 63.27) (end 105.958537 63.27) (width 0.2) (layer "B.Cu") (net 20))
 (segment (start 111.175 68.65) (end 111.175 62) (width 0.2) (layer "F.Cu") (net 19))
 (via (at 111.175 62) (size 0.4) (drill 0.3) (layers "F.Cu" "B.Cu") (free) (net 19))
 (via (at 105.85 62) (size 0.8) (drill 0.6) (layers "F.Cu" "B.Cu") (free) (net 19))
 (segment (start 111.175 62) (end 105.958244 62) (width 0.2) (layer "B.Cu") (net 19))
 (segment (start 110.675 68.65) (end 110.675 60.73) (width 0.2) (layer "F.Cu") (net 18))
 (via (at 105.85 60.73) (size 0.8) (drill 0.6) (layers "F.Cu" "B.Cu") (free) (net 18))
 (via (at 110.675 60.73) (size 0.4) (drill 0.3) (layers "F.Cu" "B.Cu") (free) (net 18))
 (segment (start 110.675 60.73) (end 105.957951 60.73) (width 0.2) (layer "B.Cu") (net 18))
 (segment (start 110.175 68.65) (end 110.175 59.46) (width 0.2) (layer "F.Cu") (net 17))
 (via (at 105.85 59.46) (size 0.8) (drill 0.6) (layers "F.Cu" "B.Cu") (free) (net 17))
 (via (at 110.175 59.46) (size 0.4) (drill 0.3) (layers "F.Cu" "B.Cu") (free) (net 17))
 (segment (start 110.175 59.46) (end 105.957658 59.46) (width 0.2) (layer "B.Cu") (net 17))
 (segment (start 110.175 49.15) (end 110.175 58.19) (width 0.2) (layer "F.Cu") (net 16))
 (via (at 110.175 58.19) (size 0.4) (drill 0.3) (layers "F.Cu" "B.Cu") (free) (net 16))
 (via (at 105.85 58.19) (size 0.8) (drill 0.6) (layers "F.Cu" "B.Cu") (free) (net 16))
 (segment (start 110.175 58.19) (end 105.957365 58.19) (width 0.2) (layer "B.Cu") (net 16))
 (segment (start 110.675 49.15) (end 110.675 56.92) (width 0.2) (layer "F.Cu") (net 15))
 (via (at 110.675 56.92) (size 0.4) (drill 0.3) (layers "F.Cu" "B.Cu") (free) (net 15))
 (via (at 105.85 56.92) (size 0.8) (drill 0.6) (layers "F.Cu" "B.Cu") (free) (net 15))
 (segment (start 110.675 56.92) (end 105.957072 56.92) (width 0.2) (layer "B.Cu") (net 15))
 (segment (start 111.175 49.15) (end 111.175 55.65) (width 0.2) (layer "F.Cu") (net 14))
 (via (at 105.85 55.65) (size 0.8) (drill 0.6) (layers "F.Cu" "B.Cu") (free) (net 14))
 (via (at 111.175 55.65) (size 0.4) (drill 0.3) (layers "F.Cu" "B.Cu") (free) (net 14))
 (segment (start 111.175 55.65) (end 105.956779 55.65) (width 0.2) (layer "B.Cu") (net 14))
 (segment (start 111.675 49.15) (end 111.675 54.38) (width 0.2) (layer "F.Cu") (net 13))
 (via (at 105.85 54.38) (size 0.8) (drill 0.6) (layers "F.Cu" "B.Cu") (free) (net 13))
 (via (at 111.675 54.38) (size 0.4) (drill 0.3) (layers "F.Cu" "B.Cu") (free) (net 13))
 (segment (start 111.675 54.38) (end 105.956486 54.38) (width 0.2) (layer "B.Cu") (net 13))
 (segment (start 112.175 49.15) (end 112.175 53.11) (width 0.2) (layer "F.Cu") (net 12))
 (via (at 105.85 53.11) (size 0.8) (drill 0.6) (layers "F.Cu" "B.Cu") (free) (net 12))
 (via (at 112.175 53.11) (size 0.4) (drill 0.3) (layers "F.Cu" "B.Cu") (free) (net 12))
 (segment (start 112.175 53.11) (end 105.956193 53.11) (width 0.2) (layer "B.Cu") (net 12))
 (segment (start 112.675 49.15) (end 112.675 51.84) (width 0.2) (layer "F.Cu") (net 11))
 (via (at 112.675 51.84) (size 0.4) (drill 0.3) (layers "F.Cu" "B.Cu") (free) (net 11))
 (via (at 105.85 51.84) (size 0.8) (drill 0.6) (layers "F.Cu" "B.Cu") (free) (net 11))
 (segment (start 112.675 51.84) (end 105.9559 51.84) (width 0.2) (layer "B.Cu") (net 11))
 (segment (start 113.175 49.15) (end 113.175 50.57) (width 0.2) (layer "F.Cu") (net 10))
 (via (at 105.85 50.57) (size 0.8) (drill 0.6) (layers "F.Cu" "B.Cu") (free) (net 10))
 (via (at 113.175 50.57) (size 0.4) (drill 0.3) (layers "F.Cu" "B.Cu") (free) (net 10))
 (segment (start 113.175 50.57) (end 105.955607 50.57) (width 0.2) (layer "B.Cu") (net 10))
 (segment (start 114.675 55.1425) (end 110.9875 58.83) (width 0.2) (layer "F.Cu") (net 1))
 (segment (start 109.39 58.8) (end 109.42 58.83) (width 0.2) (layer "F.Cu") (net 1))
 (segment (start 109.39 57.1925) (end 109.39 58.8) (width 0.2) (layer "F.Cu") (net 1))
 (segment (start 110.9875 58.83) (end 109.42 58.83) (width 0.2) (layer "F.Cu") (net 1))
 (segment (start 114.675 49.175) (end 114.675 55.1425) (width 0.2) (layer "F.Cu") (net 1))
 (segment (start 109.42 58.83) (end 108.13 58.83) (width 0.2) (layer "F.Cu") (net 1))
 (segment (start 109.39 57.1925) (end 108.05 55.8525) (width 0.2) (layer "F.Cu") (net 1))
 (via (at 105.85 49.3) (size 0.8) (drill 0.6) (layers "F.Cu" "B.Cu") (free) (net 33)))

